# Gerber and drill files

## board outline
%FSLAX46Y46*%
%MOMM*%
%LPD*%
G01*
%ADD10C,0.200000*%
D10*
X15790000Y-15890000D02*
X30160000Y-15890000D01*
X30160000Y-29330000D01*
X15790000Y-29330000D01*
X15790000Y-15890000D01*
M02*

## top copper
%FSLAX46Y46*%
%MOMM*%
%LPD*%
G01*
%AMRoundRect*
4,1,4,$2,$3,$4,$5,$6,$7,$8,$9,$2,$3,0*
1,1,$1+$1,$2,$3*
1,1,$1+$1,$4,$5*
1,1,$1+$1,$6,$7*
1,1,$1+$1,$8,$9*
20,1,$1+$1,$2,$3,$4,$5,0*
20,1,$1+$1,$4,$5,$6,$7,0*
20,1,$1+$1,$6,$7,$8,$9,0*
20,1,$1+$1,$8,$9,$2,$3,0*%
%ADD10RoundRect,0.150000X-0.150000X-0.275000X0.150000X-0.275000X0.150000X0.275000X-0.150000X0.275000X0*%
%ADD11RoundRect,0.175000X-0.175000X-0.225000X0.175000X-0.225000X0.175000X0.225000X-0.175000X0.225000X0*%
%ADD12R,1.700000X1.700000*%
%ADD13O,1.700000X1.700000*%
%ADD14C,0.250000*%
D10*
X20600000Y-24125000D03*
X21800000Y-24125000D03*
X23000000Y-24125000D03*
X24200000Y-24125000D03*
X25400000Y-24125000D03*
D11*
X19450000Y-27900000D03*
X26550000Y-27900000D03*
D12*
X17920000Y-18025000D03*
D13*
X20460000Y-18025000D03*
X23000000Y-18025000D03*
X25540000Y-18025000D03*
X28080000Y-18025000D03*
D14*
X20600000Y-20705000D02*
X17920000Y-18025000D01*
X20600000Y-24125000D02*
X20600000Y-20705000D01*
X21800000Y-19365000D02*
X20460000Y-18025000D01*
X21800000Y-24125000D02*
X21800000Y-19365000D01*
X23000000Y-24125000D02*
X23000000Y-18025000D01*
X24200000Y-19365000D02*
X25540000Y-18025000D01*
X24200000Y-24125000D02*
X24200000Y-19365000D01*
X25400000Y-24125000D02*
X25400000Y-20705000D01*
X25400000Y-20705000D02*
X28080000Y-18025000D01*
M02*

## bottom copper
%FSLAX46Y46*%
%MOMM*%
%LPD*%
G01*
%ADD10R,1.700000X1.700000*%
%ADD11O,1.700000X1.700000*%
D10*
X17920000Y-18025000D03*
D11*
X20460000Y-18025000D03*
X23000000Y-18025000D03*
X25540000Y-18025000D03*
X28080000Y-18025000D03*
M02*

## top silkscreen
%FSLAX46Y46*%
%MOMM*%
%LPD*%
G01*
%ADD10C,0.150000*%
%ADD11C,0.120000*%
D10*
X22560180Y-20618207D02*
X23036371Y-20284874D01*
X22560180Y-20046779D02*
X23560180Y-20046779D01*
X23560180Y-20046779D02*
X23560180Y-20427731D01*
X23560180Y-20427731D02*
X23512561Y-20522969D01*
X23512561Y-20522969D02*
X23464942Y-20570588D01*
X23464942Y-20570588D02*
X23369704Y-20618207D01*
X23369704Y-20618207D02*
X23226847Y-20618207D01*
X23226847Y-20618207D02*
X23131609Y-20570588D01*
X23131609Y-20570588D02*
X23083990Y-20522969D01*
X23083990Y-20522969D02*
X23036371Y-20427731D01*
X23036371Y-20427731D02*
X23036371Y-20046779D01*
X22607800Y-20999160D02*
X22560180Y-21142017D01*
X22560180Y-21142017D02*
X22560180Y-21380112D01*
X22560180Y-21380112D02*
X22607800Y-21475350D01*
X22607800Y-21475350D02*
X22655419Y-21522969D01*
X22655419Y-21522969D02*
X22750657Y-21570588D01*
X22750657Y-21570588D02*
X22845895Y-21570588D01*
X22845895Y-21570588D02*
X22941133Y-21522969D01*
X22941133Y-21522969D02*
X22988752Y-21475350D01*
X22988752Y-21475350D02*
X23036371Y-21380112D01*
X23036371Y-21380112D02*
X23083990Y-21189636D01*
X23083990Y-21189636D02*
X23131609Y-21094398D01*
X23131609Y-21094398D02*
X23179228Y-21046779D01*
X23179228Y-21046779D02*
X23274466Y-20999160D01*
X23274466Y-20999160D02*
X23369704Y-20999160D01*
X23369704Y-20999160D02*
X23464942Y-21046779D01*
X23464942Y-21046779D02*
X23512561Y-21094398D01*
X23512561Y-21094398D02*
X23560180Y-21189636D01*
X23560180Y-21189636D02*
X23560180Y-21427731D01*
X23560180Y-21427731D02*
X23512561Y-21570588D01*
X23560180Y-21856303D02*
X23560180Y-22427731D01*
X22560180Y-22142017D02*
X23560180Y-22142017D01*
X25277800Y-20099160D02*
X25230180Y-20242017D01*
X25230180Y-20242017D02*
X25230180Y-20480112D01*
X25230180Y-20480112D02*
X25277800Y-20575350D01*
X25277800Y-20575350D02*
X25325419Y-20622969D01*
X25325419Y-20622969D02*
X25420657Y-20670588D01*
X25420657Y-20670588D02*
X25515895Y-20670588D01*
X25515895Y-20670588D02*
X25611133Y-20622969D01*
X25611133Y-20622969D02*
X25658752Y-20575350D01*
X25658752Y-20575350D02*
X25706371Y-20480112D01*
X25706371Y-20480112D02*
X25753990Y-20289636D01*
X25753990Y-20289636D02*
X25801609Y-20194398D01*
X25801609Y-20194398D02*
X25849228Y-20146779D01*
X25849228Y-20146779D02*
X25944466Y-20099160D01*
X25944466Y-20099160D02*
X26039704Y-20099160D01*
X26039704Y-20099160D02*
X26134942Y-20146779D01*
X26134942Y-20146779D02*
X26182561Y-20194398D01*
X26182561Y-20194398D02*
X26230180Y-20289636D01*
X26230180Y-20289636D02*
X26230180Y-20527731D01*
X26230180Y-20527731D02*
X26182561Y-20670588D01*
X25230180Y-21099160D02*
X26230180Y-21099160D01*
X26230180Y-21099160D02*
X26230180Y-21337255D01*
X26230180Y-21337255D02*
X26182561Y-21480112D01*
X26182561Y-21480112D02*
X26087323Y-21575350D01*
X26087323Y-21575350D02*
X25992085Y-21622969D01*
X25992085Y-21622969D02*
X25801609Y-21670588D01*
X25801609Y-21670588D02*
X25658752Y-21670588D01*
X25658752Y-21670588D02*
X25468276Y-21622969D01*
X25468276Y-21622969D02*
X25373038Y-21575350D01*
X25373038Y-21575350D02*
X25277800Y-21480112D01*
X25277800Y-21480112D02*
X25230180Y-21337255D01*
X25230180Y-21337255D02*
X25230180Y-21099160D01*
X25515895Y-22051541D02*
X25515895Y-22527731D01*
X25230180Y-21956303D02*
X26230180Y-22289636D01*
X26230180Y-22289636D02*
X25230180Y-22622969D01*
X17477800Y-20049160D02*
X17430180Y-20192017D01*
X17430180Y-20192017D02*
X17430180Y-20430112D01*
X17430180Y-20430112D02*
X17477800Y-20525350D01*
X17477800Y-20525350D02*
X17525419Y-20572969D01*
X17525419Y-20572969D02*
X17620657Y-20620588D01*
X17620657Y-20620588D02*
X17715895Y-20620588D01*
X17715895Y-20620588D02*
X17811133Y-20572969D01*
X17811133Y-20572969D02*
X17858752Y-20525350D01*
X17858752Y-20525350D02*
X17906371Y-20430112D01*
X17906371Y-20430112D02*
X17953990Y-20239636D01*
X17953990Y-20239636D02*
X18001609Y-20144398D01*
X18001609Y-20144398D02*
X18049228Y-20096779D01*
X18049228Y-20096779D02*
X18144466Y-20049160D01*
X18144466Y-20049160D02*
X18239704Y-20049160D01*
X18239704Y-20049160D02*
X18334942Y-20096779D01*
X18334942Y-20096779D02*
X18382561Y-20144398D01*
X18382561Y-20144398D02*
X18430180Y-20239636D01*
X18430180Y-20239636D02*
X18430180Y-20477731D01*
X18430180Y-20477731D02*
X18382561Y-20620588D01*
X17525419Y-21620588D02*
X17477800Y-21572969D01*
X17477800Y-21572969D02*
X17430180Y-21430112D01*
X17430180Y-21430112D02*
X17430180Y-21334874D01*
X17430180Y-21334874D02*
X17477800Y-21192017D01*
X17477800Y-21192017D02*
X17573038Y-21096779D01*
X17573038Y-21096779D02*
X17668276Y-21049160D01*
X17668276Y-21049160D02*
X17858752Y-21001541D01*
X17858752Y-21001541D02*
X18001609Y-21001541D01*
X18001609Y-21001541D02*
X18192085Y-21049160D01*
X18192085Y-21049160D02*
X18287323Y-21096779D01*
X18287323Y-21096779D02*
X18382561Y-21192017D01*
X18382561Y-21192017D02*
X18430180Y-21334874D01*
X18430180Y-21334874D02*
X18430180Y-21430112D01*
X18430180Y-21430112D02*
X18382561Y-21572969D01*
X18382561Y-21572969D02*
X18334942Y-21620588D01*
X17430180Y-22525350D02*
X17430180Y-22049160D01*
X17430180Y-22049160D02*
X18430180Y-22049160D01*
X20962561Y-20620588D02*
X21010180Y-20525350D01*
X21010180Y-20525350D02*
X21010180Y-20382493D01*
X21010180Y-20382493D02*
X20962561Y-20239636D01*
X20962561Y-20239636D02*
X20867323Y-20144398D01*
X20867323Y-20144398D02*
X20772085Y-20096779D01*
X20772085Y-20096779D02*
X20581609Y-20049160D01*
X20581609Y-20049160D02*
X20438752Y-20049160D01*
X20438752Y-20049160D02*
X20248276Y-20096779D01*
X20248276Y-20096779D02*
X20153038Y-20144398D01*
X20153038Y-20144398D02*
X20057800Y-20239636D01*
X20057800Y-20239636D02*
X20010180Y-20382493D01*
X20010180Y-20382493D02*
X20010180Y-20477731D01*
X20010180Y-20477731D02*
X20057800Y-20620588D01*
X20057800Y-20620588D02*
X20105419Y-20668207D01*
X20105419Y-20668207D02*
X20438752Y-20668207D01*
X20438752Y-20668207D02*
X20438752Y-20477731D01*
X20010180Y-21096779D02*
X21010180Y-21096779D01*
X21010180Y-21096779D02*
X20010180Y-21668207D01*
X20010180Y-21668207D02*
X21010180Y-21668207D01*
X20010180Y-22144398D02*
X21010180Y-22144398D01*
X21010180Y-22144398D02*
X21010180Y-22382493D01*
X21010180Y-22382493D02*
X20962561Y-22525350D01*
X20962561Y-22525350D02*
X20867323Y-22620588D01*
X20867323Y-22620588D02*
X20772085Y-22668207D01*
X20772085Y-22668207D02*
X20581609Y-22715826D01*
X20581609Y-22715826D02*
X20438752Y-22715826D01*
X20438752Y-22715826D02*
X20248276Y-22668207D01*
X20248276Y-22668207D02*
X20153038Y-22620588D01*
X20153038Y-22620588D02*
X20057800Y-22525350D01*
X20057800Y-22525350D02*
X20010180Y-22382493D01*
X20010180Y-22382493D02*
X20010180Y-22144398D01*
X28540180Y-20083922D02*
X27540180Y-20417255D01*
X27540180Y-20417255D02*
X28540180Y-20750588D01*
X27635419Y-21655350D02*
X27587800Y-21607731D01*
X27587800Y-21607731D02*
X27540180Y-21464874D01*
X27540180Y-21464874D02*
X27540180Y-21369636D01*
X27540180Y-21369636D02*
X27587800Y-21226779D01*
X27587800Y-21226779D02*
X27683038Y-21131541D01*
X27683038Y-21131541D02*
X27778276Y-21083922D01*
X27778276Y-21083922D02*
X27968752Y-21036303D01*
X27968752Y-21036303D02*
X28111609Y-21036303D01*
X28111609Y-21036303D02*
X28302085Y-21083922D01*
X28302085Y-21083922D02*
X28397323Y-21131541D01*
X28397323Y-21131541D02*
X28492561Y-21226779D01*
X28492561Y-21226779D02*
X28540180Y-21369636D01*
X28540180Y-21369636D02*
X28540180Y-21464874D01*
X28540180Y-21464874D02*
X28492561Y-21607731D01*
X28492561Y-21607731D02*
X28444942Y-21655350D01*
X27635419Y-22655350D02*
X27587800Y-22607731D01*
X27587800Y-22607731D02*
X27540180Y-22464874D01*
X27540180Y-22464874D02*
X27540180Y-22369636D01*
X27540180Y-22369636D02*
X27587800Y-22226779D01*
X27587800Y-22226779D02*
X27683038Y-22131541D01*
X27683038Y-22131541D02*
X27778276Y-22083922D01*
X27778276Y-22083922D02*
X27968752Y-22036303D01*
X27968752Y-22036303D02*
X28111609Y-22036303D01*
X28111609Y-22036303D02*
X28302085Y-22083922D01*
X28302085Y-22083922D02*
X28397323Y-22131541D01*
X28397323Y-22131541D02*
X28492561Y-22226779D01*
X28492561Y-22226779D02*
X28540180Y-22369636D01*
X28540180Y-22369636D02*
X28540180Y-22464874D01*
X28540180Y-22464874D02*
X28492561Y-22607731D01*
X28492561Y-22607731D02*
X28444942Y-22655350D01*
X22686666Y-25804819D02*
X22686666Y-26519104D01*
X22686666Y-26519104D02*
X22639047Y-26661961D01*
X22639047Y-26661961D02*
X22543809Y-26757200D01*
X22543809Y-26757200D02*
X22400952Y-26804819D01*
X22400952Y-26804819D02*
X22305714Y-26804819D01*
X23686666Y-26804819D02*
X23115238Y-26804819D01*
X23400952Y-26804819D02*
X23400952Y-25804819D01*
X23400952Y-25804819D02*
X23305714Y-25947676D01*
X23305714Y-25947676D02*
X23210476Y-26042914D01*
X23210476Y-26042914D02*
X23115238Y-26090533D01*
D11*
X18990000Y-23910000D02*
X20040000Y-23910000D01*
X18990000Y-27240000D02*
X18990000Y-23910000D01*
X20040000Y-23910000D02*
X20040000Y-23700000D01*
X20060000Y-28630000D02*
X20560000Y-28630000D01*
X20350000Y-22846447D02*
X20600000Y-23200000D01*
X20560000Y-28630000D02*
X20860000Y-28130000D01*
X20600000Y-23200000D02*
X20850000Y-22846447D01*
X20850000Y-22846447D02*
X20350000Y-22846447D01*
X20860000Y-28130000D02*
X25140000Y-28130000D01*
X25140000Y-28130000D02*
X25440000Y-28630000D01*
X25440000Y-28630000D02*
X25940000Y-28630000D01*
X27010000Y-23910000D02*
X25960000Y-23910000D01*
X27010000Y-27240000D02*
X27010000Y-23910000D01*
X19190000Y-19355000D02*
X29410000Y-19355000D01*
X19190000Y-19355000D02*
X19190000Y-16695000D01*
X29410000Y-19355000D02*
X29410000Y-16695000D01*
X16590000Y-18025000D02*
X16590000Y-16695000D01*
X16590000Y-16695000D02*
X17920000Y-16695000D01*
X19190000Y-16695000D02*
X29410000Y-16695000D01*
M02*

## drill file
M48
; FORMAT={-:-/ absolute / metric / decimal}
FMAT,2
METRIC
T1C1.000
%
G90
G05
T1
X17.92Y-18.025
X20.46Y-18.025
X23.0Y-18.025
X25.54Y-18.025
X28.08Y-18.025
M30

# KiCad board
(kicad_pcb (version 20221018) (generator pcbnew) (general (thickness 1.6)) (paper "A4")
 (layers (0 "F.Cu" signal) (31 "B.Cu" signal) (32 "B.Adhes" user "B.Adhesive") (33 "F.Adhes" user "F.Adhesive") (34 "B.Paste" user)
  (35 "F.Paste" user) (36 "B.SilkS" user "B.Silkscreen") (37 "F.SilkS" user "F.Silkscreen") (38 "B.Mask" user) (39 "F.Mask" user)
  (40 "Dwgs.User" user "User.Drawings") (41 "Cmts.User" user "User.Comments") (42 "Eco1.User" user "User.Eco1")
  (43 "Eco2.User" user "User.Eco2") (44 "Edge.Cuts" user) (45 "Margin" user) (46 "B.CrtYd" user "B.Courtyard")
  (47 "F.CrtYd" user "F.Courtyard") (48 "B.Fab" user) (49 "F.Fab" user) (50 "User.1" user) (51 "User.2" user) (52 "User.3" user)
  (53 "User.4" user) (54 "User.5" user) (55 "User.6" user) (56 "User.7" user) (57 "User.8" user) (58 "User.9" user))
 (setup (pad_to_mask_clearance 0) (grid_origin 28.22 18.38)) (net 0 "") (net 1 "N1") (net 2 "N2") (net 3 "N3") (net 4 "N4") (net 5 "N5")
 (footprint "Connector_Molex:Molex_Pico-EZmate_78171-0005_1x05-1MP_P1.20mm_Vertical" (layer "F.Cu") (at 23 26)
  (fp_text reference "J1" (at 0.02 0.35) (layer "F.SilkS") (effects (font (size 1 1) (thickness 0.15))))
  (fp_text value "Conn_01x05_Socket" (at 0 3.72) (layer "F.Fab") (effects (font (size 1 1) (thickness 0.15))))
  (fp_line (start -4.01 -2.09) (end -2.96 -2.09) (stroke (width 0.12) (type solid)) (layer "F.SilkS"))
  (fp_line (start -4.01 1.24) (end -4.01 -2.09) (stroke (width 0.12) (type solid)) (layer "F.SilkS"))
  (fp_line (start -2.96 -2.09) (end -2.96 -2.3) (stroke (width 0.12) (type solid)) (layer "F.SilkS"))
  (fp_line (start -2.94 2.63) (end -2.44 2.63) (stroke (width 0.12) (type solid)) (layer "F.SilkS"))
  (fp_line (start -2.65 -3.153553) (end -2.4 -2.8) (stroke (width 0.12) (type solid)) (layer "F.SilkS"))
  (fp_line (start -2.44 2.63) (end -2.14 2.13) (stroke (width 0.12) (type solid)) (layer "F.SilkS"))
  (fp_line (start -2.4 -2.8) (end -2.15 -3.153553) (stroke (width 0.12) (type solid)) (layer "F.SilkS"))
  (fp_line (start -2.15 -3.153553) (end -2.65 -3.153553) (stroke (width 0.12) (type solid)) (layer "F.SilkS"))
  (fp_line (start -2.14 2.13) (end 2.14 2.13) (stroke (width 0.12) (type solid)) (layer "F.SilkS"))
  (fp_line (start 2.14 2.13) (end 2.44 2.63) (stroke (width 0.12) (type solid)) (layer "F.SilkS"))
  (fp_line (start 2.44 2.63) (end 2.94 2.63) (stroke (width 0.12) (type solid)) (layer "F.SilkS"))
  (fp_line (start 4.01 -2.09) (end 2.96 -2.09) (stroke (width 0.12) (type solid)) (layer "F.SilkS"))
  (fp_line (start 4.01 1.24) (end 4.01 -2.09) (stroke (width 0.12) (type solid)) (layer "F.SilkS"))
  (pad "1" smd roundrect (at -2.4 -1.875) (size 0.6 0.85) (layers "F.Cu" "F.Paste" "F.Mask") (roundrect_rratio 0.25) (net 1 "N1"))
  (pad "2" smd roundrect (at -1.2 -1.875) (size 0.6 0.85) (layers "F.Cu" "F.Paste" "F.Mask") (roundrect_rratio 0.25) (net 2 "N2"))
  (pad "3" smd roundrect (at 0 -1.875) (size 0.6 0.85) (layers "F.Cu" "F.Paste" "F.Mask") (roundrect_rratio 0.25) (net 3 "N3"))
  (pad "4" smd roundrect (at 1.2 -1.875) (size 0.6 0.85) (layers "F.Cu" "F.Paste" "F.Mask") (roundrect_rratio 0.25) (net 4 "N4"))
  (pad "5" smd roundrect (at 2.4 -1.875) (size 0.6 0.85) (layers "F.Cu" "F.Paste" "F.Mask") (roundrect_rratio 0.25) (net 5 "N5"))
  (pad "MP" smd roundrect (at -3.55 1.9) (size 0.7 0.8) (layers "F.Cu" "F.Paste" "F.Mask") (roundrect_rratio 0.25))
  (pad "MP" smd roundrect (at 3.55 1.9) (size 0.7 0.8) (layers "F.Cu" "F.Paste" "F.Mask") (roundrect_rratio 0.25)))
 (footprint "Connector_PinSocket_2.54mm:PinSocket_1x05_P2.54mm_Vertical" (layer "F.Cu") (at 17.92 18.025 90)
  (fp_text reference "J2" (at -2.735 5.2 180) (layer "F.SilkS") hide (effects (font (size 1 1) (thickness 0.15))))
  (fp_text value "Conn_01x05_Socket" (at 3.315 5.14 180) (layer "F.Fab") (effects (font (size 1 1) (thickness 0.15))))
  (fp_line (start -1.33 1.27) (end -1.33 11.49) (stroke (width 0.12) (type solid)) (layer "F.SilkS"))
  (fp_line (start -1.33 1.27) (end 1.33 1.27) (stroke (width 0.12) (type solid)) (layer "F.SilkS"))
  (fp_line (start -1.33 11.49) (end 1.33 11.49) (stroke (width 0.12) (type solid)) (layer "F.SilkS"))
  (fp_line (start 0 -1.33) (end 1.33 -1.33) (stroke (width 0.12) (type solid)) (layer "F.SilkS"))
  (fp_line (start 1.33 -1.33) (end 1.33 0) (stroke (width 0.12) (type solid)) (layer "F.SilkS"))
  (fp_line (start 1.33 1.27) (end 1.33 11.49) (stroke (width 0.12) (type solid)) (layer "F.SilkS"))
  (pad "1" thru_hole rect (at 0 0 90) (size 1.7 1.7) (drill 1) (layers "*.Cu" "*.Mask") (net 1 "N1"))
  (pad "2" thru_hole oval (at 0 2.54 90) (size 1.7 1.7) (drill 1) (layers "*.Cu" "*.Mask") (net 2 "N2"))
  (pad "3" thru_hole oval (at 0 5.08 90) (size 1.7 1.7) (drill 1) (layers "*.Cu" "*.Mask") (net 3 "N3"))
  (pad "4" thru_hole oval (at 0 7.62 90) (size 1.7 1.7) (drill 1) (layers "*.Cu" "*.Mask") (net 4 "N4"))
  (pad "5" thru_hole oval (at 0 10.16 90) (size 1.7 1.7) (drill 1) (layers "*.Cu" "*.Mask") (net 5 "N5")))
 (gr_rect (start 15.79 15.89) (end 30.16 29.33) (stroke (width 0.2) (type default)) (fill none) (layer "Edge.Cuts"))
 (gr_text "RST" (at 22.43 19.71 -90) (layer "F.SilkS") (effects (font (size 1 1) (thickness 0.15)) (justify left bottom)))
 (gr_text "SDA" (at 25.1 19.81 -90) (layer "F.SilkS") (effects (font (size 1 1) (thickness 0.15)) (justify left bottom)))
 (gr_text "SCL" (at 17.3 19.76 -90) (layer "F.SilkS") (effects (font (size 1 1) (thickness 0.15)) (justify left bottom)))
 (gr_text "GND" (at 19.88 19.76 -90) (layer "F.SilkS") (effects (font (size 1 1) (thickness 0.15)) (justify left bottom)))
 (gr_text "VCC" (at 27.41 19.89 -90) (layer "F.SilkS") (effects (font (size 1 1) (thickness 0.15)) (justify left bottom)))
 (segment (start 20.6 20.705) (end 17.92 18.025) (width 0.25) (layer "F.Cu") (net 1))
 (segment (start 20.6 24.125) (end 20.6 20.705) (width 0.25) (layer "F.Cu") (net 1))
 (segment (start 21.8 19.365) (end 20.46 18.025) (width 0.25) (layer "F.Cu") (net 2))
 (segment (start 21.8 24.125) (end 21.8 19.365) (width 0.25) (layer "F.Cu") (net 2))
 (segment (start 23 24.125) (end 23 18.025) (width 0.25) (layer "F.Cu") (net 3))
 (segment (start 24.2 19.365) (end 25.54 18.025) (width 0.25) (layer "F.Cu") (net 4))
 (segment (start 24.2 24.125) (end 24.2 19.365) (width 0.25) (layer "F.Cu") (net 4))
 (segment (start 25.4 24.125) (end 25.4 20.705) (width 0.25) (layer "F.Cu") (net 5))
 (segment (start 25.4 20.705) (end 28.08 18.025) (width 0.25) (layer "F.Cu") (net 5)))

